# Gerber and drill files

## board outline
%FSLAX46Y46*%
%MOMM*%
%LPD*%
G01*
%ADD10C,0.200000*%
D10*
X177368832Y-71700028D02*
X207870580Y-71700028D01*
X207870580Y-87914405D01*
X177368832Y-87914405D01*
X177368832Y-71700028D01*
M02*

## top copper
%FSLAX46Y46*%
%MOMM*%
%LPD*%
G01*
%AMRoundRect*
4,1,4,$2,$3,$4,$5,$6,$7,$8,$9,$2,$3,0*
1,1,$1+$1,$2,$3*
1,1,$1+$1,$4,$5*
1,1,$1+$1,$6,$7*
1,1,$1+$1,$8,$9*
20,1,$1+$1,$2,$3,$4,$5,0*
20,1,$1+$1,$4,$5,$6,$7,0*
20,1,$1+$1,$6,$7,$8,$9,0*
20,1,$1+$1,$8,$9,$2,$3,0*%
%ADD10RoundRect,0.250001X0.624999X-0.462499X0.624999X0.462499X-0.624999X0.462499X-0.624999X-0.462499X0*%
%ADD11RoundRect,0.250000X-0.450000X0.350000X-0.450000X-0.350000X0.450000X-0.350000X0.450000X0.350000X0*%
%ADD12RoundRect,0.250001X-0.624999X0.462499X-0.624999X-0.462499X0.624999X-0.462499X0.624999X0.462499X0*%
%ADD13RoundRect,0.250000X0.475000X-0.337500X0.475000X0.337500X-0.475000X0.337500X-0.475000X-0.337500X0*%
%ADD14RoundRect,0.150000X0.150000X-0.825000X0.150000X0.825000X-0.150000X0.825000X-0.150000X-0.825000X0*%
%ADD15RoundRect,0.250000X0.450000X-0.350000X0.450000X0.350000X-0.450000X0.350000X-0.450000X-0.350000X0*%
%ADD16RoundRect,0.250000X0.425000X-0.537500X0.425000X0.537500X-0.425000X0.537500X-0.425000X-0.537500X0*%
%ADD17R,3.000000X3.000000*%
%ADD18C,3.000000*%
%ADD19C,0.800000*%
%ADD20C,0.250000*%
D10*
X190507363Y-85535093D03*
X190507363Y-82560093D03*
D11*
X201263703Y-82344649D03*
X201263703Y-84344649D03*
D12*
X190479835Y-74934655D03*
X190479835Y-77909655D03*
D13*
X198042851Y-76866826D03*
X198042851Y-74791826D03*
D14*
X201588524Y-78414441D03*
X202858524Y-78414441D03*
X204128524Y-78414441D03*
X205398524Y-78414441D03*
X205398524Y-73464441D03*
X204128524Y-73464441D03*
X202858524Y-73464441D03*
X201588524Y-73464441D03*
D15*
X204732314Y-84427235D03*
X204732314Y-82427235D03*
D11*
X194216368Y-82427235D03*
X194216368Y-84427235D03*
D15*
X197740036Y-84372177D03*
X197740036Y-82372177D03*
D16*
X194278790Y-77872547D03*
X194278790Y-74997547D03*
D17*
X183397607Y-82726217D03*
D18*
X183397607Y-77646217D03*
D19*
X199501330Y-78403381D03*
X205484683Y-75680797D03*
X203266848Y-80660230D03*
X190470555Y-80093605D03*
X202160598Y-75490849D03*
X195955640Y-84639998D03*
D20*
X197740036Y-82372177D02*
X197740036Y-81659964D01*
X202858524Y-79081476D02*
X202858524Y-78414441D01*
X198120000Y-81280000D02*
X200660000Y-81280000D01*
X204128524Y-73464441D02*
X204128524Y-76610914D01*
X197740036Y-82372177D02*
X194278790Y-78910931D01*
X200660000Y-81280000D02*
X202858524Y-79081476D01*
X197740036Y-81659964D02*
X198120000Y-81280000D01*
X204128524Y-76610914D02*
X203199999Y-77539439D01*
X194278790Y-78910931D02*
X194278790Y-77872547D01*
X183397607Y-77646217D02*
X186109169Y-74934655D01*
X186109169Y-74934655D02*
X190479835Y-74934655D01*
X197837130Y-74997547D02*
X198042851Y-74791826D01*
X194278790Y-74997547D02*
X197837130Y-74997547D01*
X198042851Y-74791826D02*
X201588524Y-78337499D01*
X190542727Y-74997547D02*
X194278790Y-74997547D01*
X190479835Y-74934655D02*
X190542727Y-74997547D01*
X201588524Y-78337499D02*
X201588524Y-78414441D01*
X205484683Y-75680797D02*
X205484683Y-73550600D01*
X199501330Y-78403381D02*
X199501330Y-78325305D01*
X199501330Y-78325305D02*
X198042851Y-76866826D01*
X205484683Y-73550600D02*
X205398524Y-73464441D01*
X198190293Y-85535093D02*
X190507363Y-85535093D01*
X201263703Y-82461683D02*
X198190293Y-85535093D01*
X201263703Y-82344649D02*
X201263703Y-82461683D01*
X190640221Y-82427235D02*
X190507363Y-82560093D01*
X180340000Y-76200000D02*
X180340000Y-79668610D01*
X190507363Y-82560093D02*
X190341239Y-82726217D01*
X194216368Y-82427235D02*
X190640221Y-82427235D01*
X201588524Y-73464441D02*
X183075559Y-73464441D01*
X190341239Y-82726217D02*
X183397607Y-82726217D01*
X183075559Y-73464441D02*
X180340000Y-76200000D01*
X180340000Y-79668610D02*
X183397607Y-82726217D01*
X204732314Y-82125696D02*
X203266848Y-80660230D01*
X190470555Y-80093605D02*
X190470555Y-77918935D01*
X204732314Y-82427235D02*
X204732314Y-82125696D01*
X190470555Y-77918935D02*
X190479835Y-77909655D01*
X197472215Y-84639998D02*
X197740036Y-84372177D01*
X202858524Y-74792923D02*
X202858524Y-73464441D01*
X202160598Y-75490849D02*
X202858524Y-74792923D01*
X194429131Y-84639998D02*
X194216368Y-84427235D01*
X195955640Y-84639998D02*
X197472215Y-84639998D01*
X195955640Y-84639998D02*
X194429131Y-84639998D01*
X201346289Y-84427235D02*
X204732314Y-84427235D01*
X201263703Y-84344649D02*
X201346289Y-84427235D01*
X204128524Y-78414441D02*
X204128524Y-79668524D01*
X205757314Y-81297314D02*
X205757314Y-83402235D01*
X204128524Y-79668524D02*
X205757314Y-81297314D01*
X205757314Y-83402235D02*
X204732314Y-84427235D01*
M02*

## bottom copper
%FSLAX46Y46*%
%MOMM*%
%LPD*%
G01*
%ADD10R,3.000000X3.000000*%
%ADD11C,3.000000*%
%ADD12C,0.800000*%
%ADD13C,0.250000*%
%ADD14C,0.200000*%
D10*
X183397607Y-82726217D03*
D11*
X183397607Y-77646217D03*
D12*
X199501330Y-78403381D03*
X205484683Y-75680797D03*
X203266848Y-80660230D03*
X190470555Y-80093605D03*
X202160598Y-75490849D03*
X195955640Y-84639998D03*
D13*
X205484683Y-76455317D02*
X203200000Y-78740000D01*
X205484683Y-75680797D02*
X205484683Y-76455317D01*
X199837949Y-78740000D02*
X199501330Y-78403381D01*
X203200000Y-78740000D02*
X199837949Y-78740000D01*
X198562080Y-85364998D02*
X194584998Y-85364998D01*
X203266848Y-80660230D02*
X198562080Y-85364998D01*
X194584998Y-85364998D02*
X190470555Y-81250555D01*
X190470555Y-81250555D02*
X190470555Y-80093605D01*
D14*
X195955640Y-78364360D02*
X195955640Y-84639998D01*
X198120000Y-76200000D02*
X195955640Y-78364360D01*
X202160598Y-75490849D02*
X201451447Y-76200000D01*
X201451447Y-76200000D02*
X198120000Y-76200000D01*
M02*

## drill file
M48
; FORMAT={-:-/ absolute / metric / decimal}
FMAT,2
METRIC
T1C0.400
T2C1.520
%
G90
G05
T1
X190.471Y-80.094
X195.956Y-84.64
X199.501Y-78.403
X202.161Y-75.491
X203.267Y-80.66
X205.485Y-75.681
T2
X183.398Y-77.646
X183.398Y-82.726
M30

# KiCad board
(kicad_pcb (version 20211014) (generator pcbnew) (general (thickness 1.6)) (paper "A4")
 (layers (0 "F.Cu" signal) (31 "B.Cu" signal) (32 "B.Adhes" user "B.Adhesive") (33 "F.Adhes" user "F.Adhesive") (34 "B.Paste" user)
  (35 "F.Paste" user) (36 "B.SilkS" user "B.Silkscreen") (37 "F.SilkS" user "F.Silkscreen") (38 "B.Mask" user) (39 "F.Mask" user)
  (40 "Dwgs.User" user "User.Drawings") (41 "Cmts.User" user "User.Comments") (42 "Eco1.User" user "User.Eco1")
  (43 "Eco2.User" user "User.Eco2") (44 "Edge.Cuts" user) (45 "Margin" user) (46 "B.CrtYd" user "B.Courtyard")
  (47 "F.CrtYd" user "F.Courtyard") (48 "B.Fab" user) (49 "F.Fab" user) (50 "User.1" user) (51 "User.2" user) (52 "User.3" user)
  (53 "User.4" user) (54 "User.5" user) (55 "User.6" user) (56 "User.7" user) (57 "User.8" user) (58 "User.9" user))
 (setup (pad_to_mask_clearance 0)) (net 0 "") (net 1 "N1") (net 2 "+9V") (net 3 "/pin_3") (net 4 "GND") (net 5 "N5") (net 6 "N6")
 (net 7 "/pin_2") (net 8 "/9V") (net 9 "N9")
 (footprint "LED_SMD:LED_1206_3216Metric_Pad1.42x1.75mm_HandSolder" (layer "F.Cu") (at 190.507363 84.047593 90)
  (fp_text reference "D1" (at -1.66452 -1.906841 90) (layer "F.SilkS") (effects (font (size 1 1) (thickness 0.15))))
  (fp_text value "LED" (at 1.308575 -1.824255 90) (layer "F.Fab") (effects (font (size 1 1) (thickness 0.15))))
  (pad "1" smd roundrect (at -1.4875 0 90) (size 1.425 1.75) (layers "F.Cu" "F.Paste" "F.Mask") (roundrect_rratio 0.175439) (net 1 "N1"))
  (pad "2" smd roundrect (at 1.4875 0 90) (size 1.425 1.75) (layers "F.Cu" "F.Paste" "F.Mask") (roundrect_rratio 0.175439) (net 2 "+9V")))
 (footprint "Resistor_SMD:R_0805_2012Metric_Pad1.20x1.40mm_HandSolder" (layer "F.Cu") (at 201.263703 83.344649 -90)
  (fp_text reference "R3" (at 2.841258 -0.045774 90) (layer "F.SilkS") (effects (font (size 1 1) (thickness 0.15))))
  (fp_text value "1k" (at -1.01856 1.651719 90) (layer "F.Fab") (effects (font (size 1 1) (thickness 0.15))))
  (pad "1" smd roundrect (at -1 0 270) (size 1.2 1.4) (layers "F.Cu" "F.Paste" "F.Mask") (roundrect_rratio 0.208333) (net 1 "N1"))
  (pad "2" smd roundrect (at 1 0 270) (size 1.2 1.4) (layers "F.Cu" "F.Paste" "F.Mask") (roundrect_rratio 0.208333) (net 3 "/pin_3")))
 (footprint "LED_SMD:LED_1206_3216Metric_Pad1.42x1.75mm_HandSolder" (layer "F.Cu") (at 190.479835 76.422155 -90)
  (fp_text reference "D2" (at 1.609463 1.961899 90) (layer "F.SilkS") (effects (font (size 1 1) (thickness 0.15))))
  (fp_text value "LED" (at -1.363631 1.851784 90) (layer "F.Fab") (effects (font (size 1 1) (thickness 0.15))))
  (pad "1" smd roundrect (at -1.4875 0 270) (size 1.425 1.75) (layers "F.Cu" "F.Paste" "F.Mask") (roundrect_rratio 0.175439) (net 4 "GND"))
  (pad "2" smd roundrect (at 1.4875 0 270) (size 1.425 1.75) (layers "F.Cu" "F.Paste" "F.Mask") (roundrect_rratio 0.175439) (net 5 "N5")))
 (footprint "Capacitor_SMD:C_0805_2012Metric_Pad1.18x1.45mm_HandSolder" (layer "F.Cu") (at 198.042851 75.829326 90)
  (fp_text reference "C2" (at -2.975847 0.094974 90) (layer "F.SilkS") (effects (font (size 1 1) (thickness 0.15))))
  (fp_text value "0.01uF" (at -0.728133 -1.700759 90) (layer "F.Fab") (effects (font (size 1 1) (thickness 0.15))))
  (pad "1" smd roundrect (at -1.0375 0 90) (size 1.175 1.45) (layers "F.Cu" "F.Paste" "F.Mask") (roundrect_rratio 0.212766) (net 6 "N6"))
  (pad "2" smd roundrect (at 1.0375 0 90) (size 1.175 1.45) (layers "F.Cu" "F.Paste" "F.Mask") (roundrect_rratio 0.212766) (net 4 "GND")))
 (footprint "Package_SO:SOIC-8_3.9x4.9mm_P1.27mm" (layer "F.Cu") (at 203.493524 75.939441 90)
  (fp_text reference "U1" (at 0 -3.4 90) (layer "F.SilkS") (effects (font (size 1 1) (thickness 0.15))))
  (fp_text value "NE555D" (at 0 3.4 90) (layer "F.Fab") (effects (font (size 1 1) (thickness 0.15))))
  (pad "1" smd roundrect (at -2.475 -1.905 90) (size 1.95 0.6) (layers "F.Cu" "F.Paste" "F.Mask") (roundrect_rratio 0.25) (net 4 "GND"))
  (pad "2" smd roundrect (at -2.475 -0.635 90) (size 1.95 0.6) (layers "F.Cu" "F.Paste" "F.Mask") (roundrect_rratio 0.25) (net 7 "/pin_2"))
  (pad "3" smd roundrect (at -2.475 0.635 90) (size 1.95 0.6) (layers "F.Cu" "F.Paste" "F.Mask") (roundrect_rratio 0.25) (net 3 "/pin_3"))
  (pad "4" smd roundrect (at -2.475 1.905 90) (size 1.95 0.6) (layers "F.Cu" "F.Paste" "F.Mask") (roundrect_rratio 0.25) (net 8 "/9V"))
  (pad "5" smd roundrect (at 2.475 1.905 90) (size 1.95 0.6) (layers "F.Cu" "F.Paste" "F.Mask") (roundrect_rratio 0.25) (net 6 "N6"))
  (pad "6" smd roundrect (at 2.475 0.635 90) (size 1.95 0.6) (layers "F.Cu" "F.Paste" "F.Mask") (roundrect_rratio 0.25) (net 7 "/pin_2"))
  (pad "7" smd roundrect (at 2.475 -0.635 90) (size 1.95 0.6) (layers "F.Cu" "F.Paste" "F.Mask") (roundrect_rratio 0.25) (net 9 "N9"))
  (pad "8" smd roundrect (at 2.475 -1.905 90) (size 1.95 0.6) (layers "F.Cu" "F.Paste" "F.Mask") (roundrect_rratio 0.25) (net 2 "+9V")))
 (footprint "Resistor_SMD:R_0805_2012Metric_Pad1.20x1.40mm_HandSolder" (layer "F.Cu") (at 204.732314 83.427235 90)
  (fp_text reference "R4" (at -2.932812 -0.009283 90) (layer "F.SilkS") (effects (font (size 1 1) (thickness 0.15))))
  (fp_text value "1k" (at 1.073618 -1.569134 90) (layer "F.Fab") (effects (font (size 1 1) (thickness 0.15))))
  (pad "1" smd roundrect (at -1 0 90) (size 1.2 1.4) (layers "F.Cu" "F.Paste" "F.Mask") (roundrect_rratio 0.208333) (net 3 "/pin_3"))
  (pad "2" smd roundrect (at 1 0 90) (size 1.2 1.4) (layers "F.Cu" "F.Paste" "F.Mask") (roundrect_rratio 0.208333) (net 5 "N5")))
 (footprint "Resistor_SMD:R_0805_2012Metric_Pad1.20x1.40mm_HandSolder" (layer "F.Cu") (at 194.216368 83.427235 -90)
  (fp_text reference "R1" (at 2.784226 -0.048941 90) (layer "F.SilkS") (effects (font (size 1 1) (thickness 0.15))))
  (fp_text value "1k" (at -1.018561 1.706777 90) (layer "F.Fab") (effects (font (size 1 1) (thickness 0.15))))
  (pad "1" smd roundrect (at -1 0 270) (size 1.2 1.4) (layers "F.Cu" "F.Paste" "F.Mask") (roundrect_rratio 0.208333) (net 2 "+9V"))
  (pad "2" smd roundrect (at 1 0 270) (size 1.2 1.4) (layers "F.Cu" "F.Paste" "F.Mask") (roundrect_rratio 0.208333) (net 9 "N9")))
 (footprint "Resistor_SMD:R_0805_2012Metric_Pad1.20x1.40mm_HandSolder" (layer "F.Cu") (at 197.740036 83.372177 90)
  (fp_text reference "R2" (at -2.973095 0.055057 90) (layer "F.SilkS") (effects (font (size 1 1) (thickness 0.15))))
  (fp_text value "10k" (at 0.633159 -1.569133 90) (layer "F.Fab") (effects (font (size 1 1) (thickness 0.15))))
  (pad "1" smd roundrect (at -1 0 90) (size 1.2 1.4) (layers "F.Cu" "F.Paste" "F.Mask") (roundrect_rratio 0.208333) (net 9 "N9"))
  (pad "2" smd roundrect (at 1 0 90) (size 1.2 1.4) (layers "F.Cu" "F.Paste" "F.Mask") (roundrect_rratio 0.208333) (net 7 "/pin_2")))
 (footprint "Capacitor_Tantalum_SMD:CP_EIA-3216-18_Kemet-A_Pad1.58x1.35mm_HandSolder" (layer "F.Cu") (at 194.27879 76.435047 90)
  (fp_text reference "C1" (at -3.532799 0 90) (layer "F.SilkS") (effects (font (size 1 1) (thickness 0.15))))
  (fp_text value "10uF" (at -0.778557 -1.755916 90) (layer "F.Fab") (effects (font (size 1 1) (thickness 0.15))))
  (pad "1" smd roundrect (at -1.4375 0 90) (size 1.575 1.35) (layers "F.Cu" "F.Paste" "F.Mask") (roundrect_rratio 0.185185) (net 7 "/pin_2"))
  (pad "2" smd roundrect (at 1.4375 0 90) (size 1.575 1.35) (layers "F.Cu" "F.Paste" "F.Mask") (roundrect_rratio 0.185185) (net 4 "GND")))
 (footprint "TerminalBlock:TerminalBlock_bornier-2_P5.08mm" (layer "F.Cu") (at 183.397607 82.726217 90)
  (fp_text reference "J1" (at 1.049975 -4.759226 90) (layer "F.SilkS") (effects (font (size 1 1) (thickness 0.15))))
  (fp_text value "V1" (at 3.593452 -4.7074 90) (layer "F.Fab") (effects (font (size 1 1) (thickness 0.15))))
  (pad "1" thru_hole rect (at 0 0 90) (size 3 3) (drill 1.52) (layers F&B.Cu *.Mask) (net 2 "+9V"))
  (pad "2" thru_hole circle (at 5.08 0 90) (size 3 3) (drill 1.52) (layers F&B.Cu *.Mask) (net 4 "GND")))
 (gr_rect (start 177.368832 71.700028) (end 207.87058 87.914405) (layer "Edge.Cuts") (width 0.2) (fill none))
 (segment (start 197.740036 82.372177) (end 197.740036 81.659964) (width 0.25) (layer "F.Cu") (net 7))
 (segment (start 202.858524 79.081476) (end 202.858524 78.414441) (width 0.25) (layer "F.Cu") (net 7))
 (segment (start 198.12 81.28) (end 200.66 81.28) (width 0.25) (layer "F.Cu") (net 7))
 (segment (start 204.128524 73.464441) (end 204.128524 76.610914) (width 0.25) (layer "F.Cu") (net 7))
 (segment (start 197.740036 82.372177) (end 194.27879 78.910931) (width 0.25) (layer "F.Cu") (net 7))
 (segment (start 200.66 81.28) (end 202.858524 79.081476) (width 0.25) (layer "F.Cu") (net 7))
 (segment (start 197.740036 81.659964) (end 198.12 81.28) (width 0.25) (layer "F.Cu") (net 7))
 (segment (start 204.128524 76.610914) (end 203.199999 77.539439) (width 0.25) (layer "F.Cu") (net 7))
 (segment (start 194.27879 78.910931) (end 194.27879 77.872547) (width 0.25) (layer "F.Cu") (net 7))
 (segment (start 183.397607 77.646217) (end 186.109169 74.934655) (width 0.25) (layer "F.Cu") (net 4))
 (segment (start 186.109169 74.934655) (end 190.479835 74.934655) (width 0.25) (layer "F.Cu") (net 4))
 (segment (start 197.83713 74.997547) (end 198.042851 74.791826) (width 0.25) (layer "F.Cu") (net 4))
 (segment (start 194.27879 74.997547) (end 197.83713 74.997547) (width 0.25) (layer "F.Cu") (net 4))
 (segment (start 198.042851 74.791826) (end 201.588524 78.337499) (width 0.25) (layer "F.Cu") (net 4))
 (segment (start 190.542727 74.997547) (end 194.27879 74.997547) (width 0.25) (layer "F.Cu") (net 4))
 (segment (start 190.479835 74.934655) (end 190.542727 74.997547) (width 0.25) (layer "F.Cu") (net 4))
 (segment (start 201.588524 78.337499) (end 201.588524 78.414441) (width 0.25) (layer "F.Cu") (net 4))
 (segment (start 205.484683 75.680797) (end 205.484683 73.5506) (width 0.25) (layer "F.Cu") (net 6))
 (segment (start 199.50133 78.403381) (end 199.50133 78.325305) (width 0.25) (layer "F.Cu") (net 6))
 (segment (start 199.50133 78.325305) (end 198.042851 76.866826) (width 0.25) (layer "F.Cu") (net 6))
 (segment (start 205.484683 73.5506) (end 205.398524 73.464441) (width 0.25) (layer "F.Cu") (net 6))
 (via (at 199.50133 78.403381) (size 0.8) (drill 0.4) (layers "F.Cu" "B.Cu") (free) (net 6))
 (via (at 205.484683 75.680797) (size 0.8) (drill 0.4) (layers "F.Cu" "B.Cu") (free) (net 6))
 (segment (start 205.484683 76.455317) (end 203.2 78.74) (width 0.25) (layer "B.Cu") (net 6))
 (segment (start 205.484683 75.680797) (end 205.484683 76.455317) (width 0.25) (layer "B.Cu") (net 6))
 (segment (start 199.837949 78.74) (end 199.50133 78.403381) (width 0.25) (layer "B.Cu") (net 6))
 (segment (start 203.2 78.74) (end 199.837949 78.74) (width 0.25) (layer "B.Cu") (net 6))
 (segment (start 198.190293 85.535093) (end 190.507363 85.535093) (width 0.25) (layer "F.Cu") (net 1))
 (segment (start 201.263703 82.461683) (end 198.190293 85.535093) (width 0.25) (layer "F.Cu") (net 1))
 (segment (start 201.263703 82.344649) (end 201.263703 82.461683) (width 0.25) (layer "F.Cu") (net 1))
 (segment (start 190.640221 82.427235) (end 190.507363 82.560093) (width 0.25) (layer "F.Cu") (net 2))
 (segment (start 180.34 76.2) (end 180.34 79.66861) (width 0.25) (layer "F.Cu") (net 2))
 (segment (start 190.507363 82.560093) (end 190.341239 82.726217) (width 0.25) (layer "F.Cu") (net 2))
 (segment (start 194.216368 82.427235) (end 190.640221 82.427235) (width 0.25) (layer "F.Cu") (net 2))
 (segment (start 201.588524 73.464441) (end 183.075559 73.464441) (width 0.25) (layer "F.Cu") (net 2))
 (segment (start 190.341239 82.726217) (end 183.397607 82.726217) (width 0.25) (layer "F.Cu") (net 2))
 (segment (start 183.075559 73.464441) (end 180.34 76.2) (width 0.25) (layer "F.Cu") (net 2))
 (segment (start 180.34 79.66861) (end 183.397607 82.726217) (width 0.25) (layer "F.Cu") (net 2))
 (segment (start 204.732314 82.125696) (end 203.266848 80.66023) (width 0.25) (layer "F.Cu") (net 5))
 (segment (start 190.470555 80.093605) (end 190.470555 77.918935) (width 0.25) (layer "F.Cu") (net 5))
 (segment (start 204.732314 82.427235) (end 204.732314 82.125696) (width 0.25) (layer "F.Cu") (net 5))
 (segment (start 190.470555 77.918935) (end 190.479835 77.909655) (width 0.25) (layer "F.Cu") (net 5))
 (via (at 203.266848 80.66023) (size 0.8) (drill 0.4) (layers "F.Cu" "B.Cu") (free) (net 5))
 (via (at 190.470555 80.093605) (size 0.8) (drill 0.4) (layers "F.Cu" "B.Cu") (free) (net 5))
 (segment (start 198.56208 85.364998) (end 194.584998 85.364998) (width 0.25) (layer "B.Cu") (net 5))
 (segment (start 203.266848 80.66023) (end 198.56208 85.364998) (width 0.25) (layer "B.Cu") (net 5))
 (segment (start 194.584998 85.364998) (end 190.470555 81.250555) (width 0.25) (layer "B.Cu") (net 5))
 (segment (start 190.470555 81.250555) (end 190.470555 80.093605) (width 0.25) (layer "B.Cu") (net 5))
 (segment (start 197.472215 84.639998) (end 197.740036 84.372177) (width 0.25) (layer "F.Cu") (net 9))
 (segment (start 202.858524 74.792923) (end 202.858524 73.464441) (width 0.25) (layer "F.Cu") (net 9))
 (segment (start 202.160598 75.490849) (end 202.858524 74.792923) (width 0.25) (layer "F.Cu") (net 9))
 (segment (start 194.429131 84.639998) (end 194.216368 84.427235) (width 0.25) (layer "F.Cu") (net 9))
 (segment (start 195.95564 84.639998) (end 197.472215 84.639998) (width 0.25) (layer "F.Cu") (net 9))
 (segment (start 195.95564 84.639998) (end 194.429131 84.639998) (width 0.25) (layer "F.Cu") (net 9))
 (via (at 202.160598 75.490849) (size 0.8) (drill 0.4) (layers "F.Cu" "B.Cu") (free) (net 9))
 (via (at 195.95564 84.639998) (size 0.8) (drill 0.4) (layers "F.Cu" "B.Cu") (free) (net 9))
 (segment (start 195.95564 78.36436) (end 195.95564 84.639998) (width 0.2) (layer "B.Cu") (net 9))
 (segment (start 198.12 76.2) (end 195.95564 78.36436) (width 0.2) (layer "B.Cu") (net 9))
 (segment (start 202.160598 75.490849) (end 201.451447 76.2) (width 0.2) (layer "B.Cu") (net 9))
 (segment (start 201.451447 76.2) (end 198.12 76.2) (width 0.2) (layer "B.Cu") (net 9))
 (segment (start 201.346289 84.427235) (end 204.732314 84.427235) (width 0.25) (layer "F.Cu") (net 3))
 (segment (start 201.263703 84.344649) (end 201.346289 84.427235) (width 0.25) (layer "F.Cu") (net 3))
 (segment (start 204.128524 78.414441) (end 204.128524 79.668524) (width 0.25) (layer "F.Cu") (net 3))
 (segment (start 205.757314 81.297314) (end 205.757314 83.402235) (width 0.25) (layer "F.Cu") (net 3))
 (segment (start 204.128524 79.668524) (end 205.757314 81.297314) (width 0.25) (layer "F.Cu") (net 3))
 (segment (start 205.757314 83.402235) (end 204.732314 84.427235) (width 0.25) (layer "F.Cu") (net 3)))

